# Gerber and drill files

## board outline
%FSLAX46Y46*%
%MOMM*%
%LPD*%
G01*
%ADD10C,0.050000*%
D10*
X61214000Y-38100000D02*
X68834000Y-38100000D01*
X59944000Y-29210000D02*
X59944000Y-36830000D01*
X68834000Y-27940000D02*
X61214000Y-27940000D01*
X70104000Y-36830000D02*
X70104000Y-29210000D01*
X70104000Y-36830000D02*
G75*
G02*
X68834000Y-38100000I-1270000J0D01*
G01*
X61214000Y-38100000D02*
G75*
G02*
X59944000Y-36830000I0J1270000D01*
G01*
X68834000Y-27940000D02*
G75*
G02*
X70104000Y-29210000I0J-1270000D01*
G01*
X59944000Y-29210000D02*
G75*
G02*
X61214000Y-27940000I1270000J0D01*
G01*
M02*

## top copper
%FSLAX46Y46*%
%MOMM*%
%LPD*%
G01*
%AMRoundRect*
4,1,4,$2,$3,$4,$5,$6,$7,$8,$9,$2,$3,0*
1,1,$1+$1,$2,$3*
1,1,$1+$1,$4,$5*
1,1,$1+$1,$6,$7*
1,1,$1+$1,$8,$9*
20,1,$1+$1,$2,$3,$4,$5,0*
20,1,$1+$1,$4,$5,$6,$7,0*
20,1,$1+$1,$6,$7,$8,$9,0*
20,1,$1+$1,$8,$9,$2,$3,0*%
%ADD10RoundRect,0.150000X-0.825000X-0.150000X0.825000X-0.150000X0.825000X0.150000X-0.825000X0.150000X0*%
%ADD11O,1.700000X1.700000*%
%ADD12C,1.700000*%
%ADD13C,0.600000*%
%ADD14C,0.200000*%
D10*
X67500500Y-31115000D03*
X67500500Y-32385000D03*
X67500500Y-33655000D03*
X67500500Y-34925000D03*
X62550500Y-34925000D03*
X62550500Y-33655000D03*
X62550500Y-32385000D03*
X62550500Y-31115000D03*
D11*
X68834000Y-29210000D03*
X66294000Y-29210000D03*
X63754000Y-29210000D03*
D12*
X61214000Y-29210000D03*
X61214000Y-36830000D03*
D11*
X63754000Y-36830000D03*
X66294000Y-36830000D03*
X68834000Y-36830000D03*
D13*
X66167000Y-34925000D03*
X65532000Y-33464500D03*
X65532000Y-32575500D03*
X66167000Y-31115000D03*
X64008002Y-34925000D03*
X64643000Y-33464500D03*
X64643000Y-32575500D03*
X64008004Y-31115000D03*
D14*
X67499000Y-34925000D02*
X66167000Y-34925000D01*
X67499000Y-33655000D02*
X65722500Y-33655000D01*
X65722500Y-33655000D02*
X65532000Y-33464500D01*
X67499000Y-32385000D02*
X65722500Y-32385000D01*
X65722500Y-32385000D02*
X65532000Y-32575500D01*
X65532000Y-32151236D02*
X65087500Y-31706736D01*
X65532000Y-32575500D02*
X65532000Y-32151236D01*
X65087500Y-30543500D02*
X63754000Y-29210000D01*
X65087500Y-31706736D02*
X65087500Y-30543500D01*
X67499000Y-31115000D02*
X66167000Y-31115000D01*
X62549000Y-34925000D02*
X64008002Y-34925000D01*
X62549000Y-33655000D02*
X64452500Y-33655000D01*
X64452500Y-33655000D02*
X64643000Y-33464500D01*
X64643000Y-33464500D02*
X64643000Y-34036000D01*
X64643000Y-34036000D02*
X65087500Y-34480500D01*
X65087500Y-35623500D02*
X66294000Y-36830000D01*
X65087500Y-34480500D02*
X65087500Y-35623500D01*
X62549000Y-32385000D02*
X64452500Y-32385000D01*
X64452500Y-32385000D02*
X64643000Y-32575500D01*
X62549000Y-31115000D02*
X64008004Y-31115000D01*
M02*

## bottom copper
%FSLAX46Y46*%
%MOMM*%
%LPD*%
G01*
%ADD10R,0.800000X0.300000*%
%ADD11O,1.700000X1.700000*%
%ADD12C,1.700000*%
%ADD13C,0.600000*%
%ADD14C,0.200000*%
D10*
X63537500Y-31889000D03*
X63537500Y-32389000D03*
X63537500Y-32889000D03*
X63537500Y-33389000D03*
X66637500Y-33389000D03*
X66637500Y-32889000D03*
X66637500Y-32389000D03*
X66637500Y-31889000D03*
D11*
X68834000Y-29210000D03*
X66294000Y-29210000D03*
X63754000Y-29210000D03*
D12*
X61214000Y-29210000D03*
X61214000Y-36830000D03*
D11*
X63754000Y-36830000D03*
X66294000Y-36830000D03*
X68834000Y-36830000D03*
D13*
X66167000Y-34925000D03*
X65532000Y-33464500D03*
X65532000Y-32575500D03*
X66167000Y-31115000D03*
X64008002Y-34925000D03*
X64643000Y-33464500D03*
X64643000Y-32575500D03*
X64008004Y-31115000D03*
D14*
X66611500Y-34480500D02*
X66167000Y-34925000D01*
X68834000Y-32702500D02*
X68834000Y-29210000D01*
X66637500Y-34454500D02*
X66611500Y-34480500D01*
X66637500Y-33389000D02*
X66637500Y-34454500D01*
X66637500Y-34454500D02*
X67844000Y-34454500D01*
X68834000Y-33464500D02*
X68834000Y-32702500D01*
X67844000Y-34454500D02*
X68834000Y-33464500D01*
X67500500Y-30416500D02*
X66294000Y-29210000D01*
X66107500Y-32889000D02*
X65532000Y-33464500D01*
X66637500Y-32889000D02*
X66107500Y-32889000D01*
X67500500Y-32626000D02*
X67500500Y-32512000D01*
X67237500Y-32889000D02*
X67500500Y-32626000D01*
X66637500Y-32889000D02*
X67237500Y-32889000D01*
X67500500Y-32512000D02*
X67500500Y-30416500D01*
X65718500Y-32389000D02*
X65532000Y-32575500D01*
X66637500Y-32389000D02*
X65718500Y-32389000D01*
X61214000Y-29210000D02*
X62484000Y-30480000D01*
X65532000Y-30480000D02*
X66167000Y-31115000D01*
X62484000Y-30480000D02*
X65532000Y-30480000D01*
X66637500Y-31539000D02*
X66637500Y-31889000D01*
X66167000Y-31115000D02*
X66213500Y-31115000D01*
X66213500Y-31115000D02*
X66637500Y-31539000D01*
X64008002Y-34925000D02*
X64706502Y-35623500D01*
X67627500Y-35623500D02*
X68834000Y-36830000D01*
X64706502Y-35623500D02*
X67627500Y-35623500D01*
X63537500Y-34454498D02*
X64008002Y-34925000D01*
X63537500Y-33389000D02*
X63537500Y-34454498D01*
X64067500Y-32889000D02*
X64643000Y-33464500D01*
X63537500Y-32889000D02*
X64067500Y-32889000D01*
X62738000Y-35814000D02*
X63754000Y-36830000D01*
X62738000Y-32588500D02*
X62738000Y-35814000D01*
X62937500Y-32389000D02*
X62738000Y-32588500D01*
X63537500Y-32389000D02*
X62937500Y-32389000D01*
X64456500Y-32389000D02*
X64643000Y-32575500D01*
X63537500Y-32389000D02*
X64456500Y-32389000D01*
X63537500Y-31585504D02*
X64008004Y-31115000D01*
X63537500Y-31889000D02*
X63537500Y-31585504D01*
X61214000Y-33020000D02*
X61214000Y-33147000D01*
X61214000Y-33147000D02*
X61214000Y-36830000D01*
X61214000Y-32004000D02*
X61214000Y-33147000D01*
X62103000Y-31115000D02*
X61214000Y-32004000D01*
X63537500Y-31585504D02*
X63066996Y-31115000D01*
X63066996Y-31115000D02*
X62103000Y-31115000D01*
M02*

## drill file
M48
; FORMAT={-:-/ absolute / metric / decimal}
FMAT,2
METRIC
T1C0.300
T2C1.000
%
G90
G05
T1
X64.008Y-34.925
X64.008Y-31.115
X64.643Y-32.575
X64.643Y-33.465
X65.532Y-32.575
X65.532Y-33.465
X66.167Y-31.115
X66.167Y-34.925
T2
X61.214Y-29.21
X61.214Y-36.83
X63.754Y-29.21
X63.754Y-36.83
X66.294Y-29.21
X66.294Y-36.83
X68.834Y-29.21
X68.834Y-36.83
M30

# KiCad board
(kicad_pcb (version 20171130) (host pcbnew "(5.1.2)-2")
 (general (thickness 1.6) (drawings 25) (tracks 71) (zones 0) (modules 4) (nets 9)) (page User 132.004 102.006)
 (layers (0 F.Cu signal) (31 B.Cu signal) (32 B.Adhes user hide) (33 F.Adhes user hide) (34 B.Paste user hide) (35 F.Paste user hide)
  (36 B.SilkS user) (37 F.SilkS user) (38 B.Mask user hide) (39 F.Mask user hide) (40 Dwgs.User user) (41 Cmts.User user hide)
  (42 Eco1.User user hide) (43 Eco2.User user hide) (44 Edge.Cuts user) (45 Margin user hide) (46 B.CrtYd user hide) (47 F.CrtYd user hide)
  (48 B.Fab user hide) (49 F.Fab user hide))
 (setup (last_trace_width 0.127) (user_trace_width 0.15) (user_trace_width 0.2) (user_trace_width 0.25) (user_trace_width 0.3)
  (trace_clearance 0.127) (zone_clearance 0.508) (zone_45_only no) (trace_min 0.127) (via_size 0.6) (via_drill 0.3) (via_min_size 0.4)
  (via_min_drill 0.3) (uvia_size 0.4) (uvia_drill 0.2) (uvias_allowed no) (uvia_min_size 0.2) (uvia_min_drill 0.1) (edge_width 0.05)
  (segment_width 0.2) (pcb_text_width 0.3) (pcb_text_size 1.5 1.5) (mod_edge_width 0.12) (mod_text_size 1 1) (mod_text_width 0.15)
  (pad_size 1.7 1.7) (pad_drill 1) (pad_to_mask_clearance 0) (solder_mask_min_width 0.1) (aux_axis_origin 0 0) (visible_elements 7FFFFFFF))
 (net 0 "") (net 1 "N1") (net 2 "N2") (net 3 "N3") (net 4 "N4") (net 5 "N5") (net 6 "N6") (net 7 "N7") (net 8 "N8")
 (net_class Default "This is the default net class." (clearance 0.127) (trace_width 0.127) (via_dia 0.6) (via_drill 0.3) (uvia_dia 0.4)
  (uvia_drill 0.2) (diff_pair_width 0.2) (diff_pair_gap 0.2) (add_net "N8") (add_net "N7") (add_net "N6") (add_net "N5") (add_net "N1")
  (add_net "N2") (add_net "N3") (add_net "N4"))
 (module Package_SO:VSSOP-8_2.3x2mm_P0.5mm (layer B.Cu) (at 65.0875 32.639 180)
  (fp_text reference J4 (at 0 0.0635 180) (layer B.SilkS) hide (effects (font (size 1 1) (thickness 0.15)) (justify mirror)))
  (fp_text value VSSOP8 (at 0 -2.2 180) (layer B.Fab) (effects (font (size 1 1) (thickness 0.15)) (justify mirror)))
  (pad 8 smd rect (at 1.55 0.75 270) (size 0.3 0.8) (layers B.Cu B.Paste B.Mask) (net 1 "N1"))
  (pad 7 smd rect (at 1.55 0.25 270) (size 0.3 0.8) (layers B.Cu B.Paste B.Mask) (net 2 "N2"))
  (pad 6 smd rect (at 1.55 -0.25 270) (size 0.3 0.8) (layers B.Cu B.Paste B.Mask) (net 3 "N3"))
  (pad 5 smd rect (at 1.55 -0.75 270) (size 0.3 0.8) (layers B.Cu B.Paste B.Mask) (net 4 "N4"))
  (pad 4 smd rect (at -1.55 -0.75 270) (size 0.3 0.8) (layers B.Cu B.Paste B.Mask) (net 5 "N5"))
  (pad 3 smd rect (at -1.55 -0.25 270) (size 0.3 0.8) (layers B.Cu B.Paste B.Mask) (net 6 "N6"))
  (pad 2 smd rect (at -1.55 0.25 270) (size 0.3 0.8) (layers B.Cu B.Paste B.Mask) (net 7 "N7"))
  (pad 1 smd rect (at -1.55 0.75 270) (size 0.3 0.8) (layers B.Cu B.Paste B.Mask) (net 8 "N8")))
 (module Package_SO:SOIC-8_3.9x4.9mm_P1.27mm (layer F.Cu) (at 65.0255 33.02)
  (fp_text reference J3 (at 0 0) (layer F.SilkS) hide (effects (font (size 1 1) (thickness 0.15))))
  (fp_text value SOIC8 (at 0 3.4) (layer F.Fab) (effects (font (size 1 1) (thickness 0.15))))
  (pad 8 smd roundrect (at 2.475 -1.905) (size 1.95 0.6) (layers F.Cu F.Paste F.Mask) (roundrect_rratio 0.25) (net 8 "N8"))
  (pad 7 smd roundrect (at 2.475 -0.635) (size 1.95 0.6) (layers F.Cu F.Paste F.Mask) (roundrect_rratio 0.25) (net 7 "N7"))
  (pad 6 smd roundrect (at 2.475 0.635) (size 1.95 0.6) (layers F.Cu F.Paste F.Mask) (roundrect_rratio 0.25) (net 6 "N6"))
  (pad 5 smd roundrect (at 2.475 1.905) (size 1.95 0.6) (layers F.Cu F.Paste F.Mask) (roundrect_rratio 0.25) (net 5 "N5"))
  (pad 4 smd roundrect (at -2.475 1.905) (size 1.95 0.6) (layers F.Cu F.Paste F.Mask) (roundrect_rratio 0.25) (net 4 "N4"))
  (pad 3 smd roundrect (at -2.475 0.635) (size 1.95 0.6) (layers F.Cu F.Paste F.Mask) (roundrect_rratio 0.25) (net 3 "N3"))
  (pad 2 smd roundrect (at -2.475 -0.635) (size 1.95 0.6) (layers F.Cu F.Paste F.Mask) (roundrect_rratio 0.25) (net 2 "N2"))
  (pad 1 smd roundrect (at -2.475 -1.905) (size 1.95 0.6) (layers F.Cu F.Paste F.Mask) (roundrect_rratio 0.25) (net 1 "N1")))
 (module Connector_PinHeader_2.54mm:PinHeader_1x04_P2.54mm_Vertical (layer F.Cu) (at 61.214 29.21 90)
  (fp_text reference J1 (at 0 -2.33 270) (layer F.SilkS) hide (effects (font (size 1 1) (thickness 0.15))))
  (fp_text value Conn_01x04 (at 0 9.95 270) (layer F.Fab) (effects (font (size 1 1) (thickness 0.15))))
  (pad 4 thru_hole oval (at 0 7.62 90) (size 1.7 1.7) (drill 1) (layers *.Cu *.Mask) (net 5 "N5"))
  (pad 3 thru_hole oval (at 0 5.08 90) (size 1.7 1.7) (drill 1) (layers *.Cu *.Mask) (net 6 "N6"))
  (pad 2 thru_hole oval (at 0 2.54 90) (size 1.7 1.7) (drill 1) (layers *.Cu *.Mask) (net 7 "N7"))
  (pad 1 thru_hole circle (at 0 0 90) (size 1.7 1.7) (drill 1) (layers *.Cu *.Mask) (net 8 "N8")))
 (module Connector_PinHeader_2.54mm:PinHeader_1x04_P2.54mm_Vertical (layer F.Cu) (at 61.214 36.83 90)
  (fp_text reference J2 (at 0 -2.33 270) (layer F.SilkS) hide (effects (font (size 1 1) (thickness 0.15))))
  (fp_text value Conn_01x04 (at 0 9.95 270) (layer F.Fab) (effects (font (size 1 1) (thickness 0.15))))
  (pad 1 thru_hole circle (at 0 0 90) (size 1.7 1.7) (drill 1) (layers *.Cu *.Mask) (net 1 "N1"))
  (pad 2 thru_hole oval (at 0 2.54 90) (size 1.7 1.7) (drill 1) (layers *.Cu *.Mask) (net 2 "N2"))
  (pad 3 thru_hole oval (at 0 5.08 90) (size 1.7 1.7) (drill 1) (layers *.Cu *.Mask) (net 3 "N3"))
  (pad 4 thru_hole oval (at 0 7.62 90) (size 1.7 1.7) (drill 1) (layers *.Cu *.Mask) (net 4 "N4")))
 (gr_line (start 61.214 38.1) (end 68.834 38.1) (layer Edge.Cuts) (width 0.05))
 (gr_line (start 59.944 29.21) (end 59.944 36.83) (layer Edge.Cuts) (width 0.05))
 (gr_line (start 68.834 27.94) (end 61.214 27.94) (layer Edge.Cuts) (width 0.05))
 (gr_line (start 70.104 36.83) (end 70.104 29.21) (layer Edge.Cuts) (width 0.05))
 (gr_arc (start 68.834 36.83) (end 68.834 38.1) (angle -90) (layer Edge.Cuts) (width 0.05))
 (gr_arc (start 61.214 36.83) (end 59.944 36.83) (angle -90) (layer Edge.Cuts) (width 0.05))
 (gr_arc (start 68.834 29.21) (end 70.104 29.21) (angle -90) (layer Edge.Cuts) (width 0.05))
 (gr_arc (start 61.214 29.21) (end 61.214 27.94) (angle -90) (layer Edge.Cuts) (width 0.05))
 (via (at 66.167 34.925) (size 0.6) (drill 0.3) (layers F.Cu B.Cu) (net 5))
 (segment (start 67.499 34.925) (end 66.167 34.925) (width 0.2) (layer F.Cu) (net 5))
 (segment (start 66.6115 34.4805) (end 66.167 34.925) (width 0.2) (layer B.Cu) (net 5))
 (segment (start 68.834 32.7025) (end 68.834 29.21) (width 0.2) (layer B.Cu) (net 5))
 (segment (start 66.6375 34.4545) (end 66.6115 34.4805) (width 0.2) (layer B.Cu) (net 5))
 (segment (start 66.6375 33.389) (end 66.6375 34.4545) (width 0.2) (layer B.Cu) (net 5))
 (segment (start 66.6375 34.4545) (end 67.844 34.4545) (width 0.2) (layer B.Cu) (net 5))
 (segment (start 68.834 33.4645) (end 68.834 32.7025) (width 0.2) (layer B.Cu) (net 5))
 (segment (start 67.844 34.4545) (end 68.834 33.4645) (width 0.2) (layer B.Cu) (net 5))
 (via (at 65.532 33.4645) (size 0.6) (drill 0.3) (layers F.Cu B.Cu) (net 6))
 (segment (start 67.499 33.655) (end 65.7225 33.655) (width 0.2) (layer F.Cu) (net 6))
 (segment (start 65.7225 33.655) (end 65.532 33.4645) (width 0.2) (layer F.Cu) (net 6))
 (segment (start 67.5005 30.4165) (end 66.294 29.21) (width 0.2) (layer B.Cu) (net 6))
 (segment (start 66.1075 32.889) (end 65.532 33.4645) (width 0.2) (layer B.Cu) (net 6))
 (segment (start 66.6375 32.889) (end 66.1075 32.889) (width 0.2) (layer B.Cu) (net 6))
 (segment (start 67.5005 32.626) (end 67.5005 32.512) (width 0.2) (layer B.Cu) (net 6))
 (segment (start 67.2375 32.889) (end 67.5005 32.626) (width 0.2) (layer B.Cu) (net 6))
 (segment (start 66.6375 32.889) (end 67.2375 32.889) (width 0.2) (layer B.Cu) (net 6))
 (segment (start 67.5005 32.512) (end 67.5005 30.4165) (width 0.2) (layer B.Cu) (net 6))
 (via (at 65.532 32.5755) (size 0.6) (drill 0.3) (layers F.Cu B.Cu) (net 7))
 (segment (start 67.499 32.385) (end 65.7225 32.385) (width 0.2) (layer F.Cu) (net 7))
 (segment (start 65.7225 32.385) (end 65.532 32.5755) (width 0.2) (layer F.Cu) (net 7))
 (segment (start 65.532 32.151236) (end 65.0875 31.706736) (width 0.2) (layer F.Cu) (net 7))
 (segment (start 65.532 32.5755) (end 65.532 32.151236) (width 0.2) (layer F.Cu) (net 7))
 (segment (start 65.0875 30.5435) (end 63.754 29.21) (width 0.2) (layer F.Cu) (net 7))
 (segment (start 65.0875 31.706736) (end 65.0875 30.5435) (width 0.2) (layer F.Cu) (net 7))
 (segment (start 65.7185 32.389) (end 65.532 32.5755) (width 0.2) (layer B.Cu) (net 7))
 (segment (start 66.6375 32.389) (end 65.7185 32.389) (width 0.2) (layer B.Cu) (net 7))
 (via (at 66.167 31.115) (size 0.6) (drill 0.3) (layers F.Cu B.Cu) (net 8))
 (segment (start 67.499 31.115) (end 66.167 31.115) (width 0.2) (layer F.Cu) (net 8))
 (segment (start 61.214 29.21) (end 62.484 30.48) (width 0.2) (layer B.Cu) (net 8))
 (segment (start 65.532 30.48) (end 66.167 31.115) (width 0.2) (layer B.Cu) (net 8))
 (segment (start 62.484 30.48) (end 65.532 30.48) (width 0.2) (layer B.Cu) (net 8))
 (segment (start 66.6375 31.539) (end 66.6375 31.889) (width 0.2) (layer B.Cu) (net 8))
 (segment (start 66.167 31.115) (end 66.2135 31.115) (width 0.2) (layer B.Cu) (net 8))
 (segment (start 66.2135 31.115) (end 66.6375 31.539) (width 0.2) (layer B.Cu) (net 8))
 (via (at 64.008002 34.925) (size 0.6) (drill 0.3) (layers F.Cu B.Cu) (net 4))
 (segment (start 62.549 34.925) (end 64.008002 34.925) (width 0.2) (layer F.Cu) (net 4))
 (segment (start 64.008002 34.925) (end 64.706502 35.6235) (width 0.2) (layer B.Cu) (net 4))
 (segment (start 67.6275 35.6235) (end 68.834 36.83) (width 0.2) (layer B.Cu) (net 4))
 (segment (start 64.706502 35.6235) (end 67.6275 35.6235) (width 0.2) (layer B.Cu) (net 4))
 (segment (start 63.5375 34.454498) (end 64.008002 34.925) (width 0.2) (layer B.Cu) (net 4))
 (segment (start 63.5375 33.389) (end 63.5375 34.454498) (width 0.2) (layer B.Cu) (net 4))
 (via (at 64.643 33.4645) (size 0.6) (drill 0.3) (layers F.Cu B.Cu) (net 3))
 (segment (start 62.549 33.655) (end 64.4525 33.655) (width 0.2) (layer F.Cu) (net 3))
 (segment (start 64.4525 33.655) (end 64.643 33.4645) (width 0.2) (layer F.Cu) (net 3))
 (segment (start 64.643 33.4645) (end 64.643 34.036) (width 0.2) (layer F.Cu) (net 3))
 (segment (start 64.643 34.036) (end 65.0875 34.4805) (width 0.2) (layer F.Cu) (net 3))
 (segment (start 65.0875 35.6235) (end 66.294 36.83) (width 0.2) (layer F.Cu) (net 3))
 (segment (start 65.0875 34.4805) (end 65.0875 35.6235) (width 0.2) (layer F.Cu) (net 3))
 (segment (start 64.0675 32.889) (end 64.643 33.4645) (width 0.2) (layer B.Cu) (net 3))
 (segment (start 63.5375 32.889) (end 64.0675 32.889) (width 0.2) (layer B.Cu) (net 3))
 (via (at 64.643 32.5755) (size 0.6) (drill 0.3) (layers F.Cu B.Cu) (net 2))
 (segment (start 62.549 32.385) (end 64.4525 32.385) (width 0.2) (layer F.Cu) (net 2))
 (segment (start 64.4525 32.385) (end 64.643 32.5755) (width 0.2) (layer F.Cu) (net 2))
 (segment (start 62.738 35.814) (end 63.754 36.83) (width 0.2) (layer B.Cu) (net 2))
 (segment (start 62.738 32.5885) (end 62.738 35.814) (width 0.2) (layer B.Cu) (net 2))
 (segment (start 62.9375 32.389) (end 62.738 32.5885) (width 0.2) (layer B.Cu) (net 2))
 (segment (start 63.5375 32.389) (end 62.9375 32.389) (width 0.2) (layer B.Cu) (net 2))
 (segment (start 64.4565 32.389) (end 64.643 32.5755) (width 0.2) (layer B.Cu) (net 2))
 (segment (start 63.5375 32.389) (end 64.4565 32.389) (width 0.2) (layer B.Cu) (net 2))
 (via (at 64.008004 31.115) (size 0.6) (drill 0.3) (layers F.Cu B.Cu) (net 1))
 (segment (start 62.549 31.115) (end 64.008004 31.115) (width 0.2) (layer F.Cu) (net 1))
 (segment (start 63.5375 31.585504) (end 64.008004 31.115) (width 0.2) (layer B.Cu) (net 1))
 (segment (start 63.5375 31.889) (end 63.5375 31.585504) (width 0.2) (layer B.Cu) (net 1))
 (segment (start 61.214 33.02) (end 61.214 33.147) (width 0.2) (layer B.Cu) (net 1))
 (segment (start 61.214 33.147) (end 61.214 36.83) (width 0.2) (layer B.Cu) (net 1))
 (segment (start 61.214 32.004) (end 61.214 33.147) (width 0.2) (layer B.Cu) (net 1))
 (segment (start 62.103 31.115) (end 61.214 32.004) (width 0.2) (layer B.Cu) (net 1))
 (segment (start 63.5375 31.585504) (end 63.066996 31.115) (width 0.2) (layer B.Cu) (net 1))
 (segment (start 63.066996 31.115) (end 62.103 31.115) (width 0.2) (layer B.Cu) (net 1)))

